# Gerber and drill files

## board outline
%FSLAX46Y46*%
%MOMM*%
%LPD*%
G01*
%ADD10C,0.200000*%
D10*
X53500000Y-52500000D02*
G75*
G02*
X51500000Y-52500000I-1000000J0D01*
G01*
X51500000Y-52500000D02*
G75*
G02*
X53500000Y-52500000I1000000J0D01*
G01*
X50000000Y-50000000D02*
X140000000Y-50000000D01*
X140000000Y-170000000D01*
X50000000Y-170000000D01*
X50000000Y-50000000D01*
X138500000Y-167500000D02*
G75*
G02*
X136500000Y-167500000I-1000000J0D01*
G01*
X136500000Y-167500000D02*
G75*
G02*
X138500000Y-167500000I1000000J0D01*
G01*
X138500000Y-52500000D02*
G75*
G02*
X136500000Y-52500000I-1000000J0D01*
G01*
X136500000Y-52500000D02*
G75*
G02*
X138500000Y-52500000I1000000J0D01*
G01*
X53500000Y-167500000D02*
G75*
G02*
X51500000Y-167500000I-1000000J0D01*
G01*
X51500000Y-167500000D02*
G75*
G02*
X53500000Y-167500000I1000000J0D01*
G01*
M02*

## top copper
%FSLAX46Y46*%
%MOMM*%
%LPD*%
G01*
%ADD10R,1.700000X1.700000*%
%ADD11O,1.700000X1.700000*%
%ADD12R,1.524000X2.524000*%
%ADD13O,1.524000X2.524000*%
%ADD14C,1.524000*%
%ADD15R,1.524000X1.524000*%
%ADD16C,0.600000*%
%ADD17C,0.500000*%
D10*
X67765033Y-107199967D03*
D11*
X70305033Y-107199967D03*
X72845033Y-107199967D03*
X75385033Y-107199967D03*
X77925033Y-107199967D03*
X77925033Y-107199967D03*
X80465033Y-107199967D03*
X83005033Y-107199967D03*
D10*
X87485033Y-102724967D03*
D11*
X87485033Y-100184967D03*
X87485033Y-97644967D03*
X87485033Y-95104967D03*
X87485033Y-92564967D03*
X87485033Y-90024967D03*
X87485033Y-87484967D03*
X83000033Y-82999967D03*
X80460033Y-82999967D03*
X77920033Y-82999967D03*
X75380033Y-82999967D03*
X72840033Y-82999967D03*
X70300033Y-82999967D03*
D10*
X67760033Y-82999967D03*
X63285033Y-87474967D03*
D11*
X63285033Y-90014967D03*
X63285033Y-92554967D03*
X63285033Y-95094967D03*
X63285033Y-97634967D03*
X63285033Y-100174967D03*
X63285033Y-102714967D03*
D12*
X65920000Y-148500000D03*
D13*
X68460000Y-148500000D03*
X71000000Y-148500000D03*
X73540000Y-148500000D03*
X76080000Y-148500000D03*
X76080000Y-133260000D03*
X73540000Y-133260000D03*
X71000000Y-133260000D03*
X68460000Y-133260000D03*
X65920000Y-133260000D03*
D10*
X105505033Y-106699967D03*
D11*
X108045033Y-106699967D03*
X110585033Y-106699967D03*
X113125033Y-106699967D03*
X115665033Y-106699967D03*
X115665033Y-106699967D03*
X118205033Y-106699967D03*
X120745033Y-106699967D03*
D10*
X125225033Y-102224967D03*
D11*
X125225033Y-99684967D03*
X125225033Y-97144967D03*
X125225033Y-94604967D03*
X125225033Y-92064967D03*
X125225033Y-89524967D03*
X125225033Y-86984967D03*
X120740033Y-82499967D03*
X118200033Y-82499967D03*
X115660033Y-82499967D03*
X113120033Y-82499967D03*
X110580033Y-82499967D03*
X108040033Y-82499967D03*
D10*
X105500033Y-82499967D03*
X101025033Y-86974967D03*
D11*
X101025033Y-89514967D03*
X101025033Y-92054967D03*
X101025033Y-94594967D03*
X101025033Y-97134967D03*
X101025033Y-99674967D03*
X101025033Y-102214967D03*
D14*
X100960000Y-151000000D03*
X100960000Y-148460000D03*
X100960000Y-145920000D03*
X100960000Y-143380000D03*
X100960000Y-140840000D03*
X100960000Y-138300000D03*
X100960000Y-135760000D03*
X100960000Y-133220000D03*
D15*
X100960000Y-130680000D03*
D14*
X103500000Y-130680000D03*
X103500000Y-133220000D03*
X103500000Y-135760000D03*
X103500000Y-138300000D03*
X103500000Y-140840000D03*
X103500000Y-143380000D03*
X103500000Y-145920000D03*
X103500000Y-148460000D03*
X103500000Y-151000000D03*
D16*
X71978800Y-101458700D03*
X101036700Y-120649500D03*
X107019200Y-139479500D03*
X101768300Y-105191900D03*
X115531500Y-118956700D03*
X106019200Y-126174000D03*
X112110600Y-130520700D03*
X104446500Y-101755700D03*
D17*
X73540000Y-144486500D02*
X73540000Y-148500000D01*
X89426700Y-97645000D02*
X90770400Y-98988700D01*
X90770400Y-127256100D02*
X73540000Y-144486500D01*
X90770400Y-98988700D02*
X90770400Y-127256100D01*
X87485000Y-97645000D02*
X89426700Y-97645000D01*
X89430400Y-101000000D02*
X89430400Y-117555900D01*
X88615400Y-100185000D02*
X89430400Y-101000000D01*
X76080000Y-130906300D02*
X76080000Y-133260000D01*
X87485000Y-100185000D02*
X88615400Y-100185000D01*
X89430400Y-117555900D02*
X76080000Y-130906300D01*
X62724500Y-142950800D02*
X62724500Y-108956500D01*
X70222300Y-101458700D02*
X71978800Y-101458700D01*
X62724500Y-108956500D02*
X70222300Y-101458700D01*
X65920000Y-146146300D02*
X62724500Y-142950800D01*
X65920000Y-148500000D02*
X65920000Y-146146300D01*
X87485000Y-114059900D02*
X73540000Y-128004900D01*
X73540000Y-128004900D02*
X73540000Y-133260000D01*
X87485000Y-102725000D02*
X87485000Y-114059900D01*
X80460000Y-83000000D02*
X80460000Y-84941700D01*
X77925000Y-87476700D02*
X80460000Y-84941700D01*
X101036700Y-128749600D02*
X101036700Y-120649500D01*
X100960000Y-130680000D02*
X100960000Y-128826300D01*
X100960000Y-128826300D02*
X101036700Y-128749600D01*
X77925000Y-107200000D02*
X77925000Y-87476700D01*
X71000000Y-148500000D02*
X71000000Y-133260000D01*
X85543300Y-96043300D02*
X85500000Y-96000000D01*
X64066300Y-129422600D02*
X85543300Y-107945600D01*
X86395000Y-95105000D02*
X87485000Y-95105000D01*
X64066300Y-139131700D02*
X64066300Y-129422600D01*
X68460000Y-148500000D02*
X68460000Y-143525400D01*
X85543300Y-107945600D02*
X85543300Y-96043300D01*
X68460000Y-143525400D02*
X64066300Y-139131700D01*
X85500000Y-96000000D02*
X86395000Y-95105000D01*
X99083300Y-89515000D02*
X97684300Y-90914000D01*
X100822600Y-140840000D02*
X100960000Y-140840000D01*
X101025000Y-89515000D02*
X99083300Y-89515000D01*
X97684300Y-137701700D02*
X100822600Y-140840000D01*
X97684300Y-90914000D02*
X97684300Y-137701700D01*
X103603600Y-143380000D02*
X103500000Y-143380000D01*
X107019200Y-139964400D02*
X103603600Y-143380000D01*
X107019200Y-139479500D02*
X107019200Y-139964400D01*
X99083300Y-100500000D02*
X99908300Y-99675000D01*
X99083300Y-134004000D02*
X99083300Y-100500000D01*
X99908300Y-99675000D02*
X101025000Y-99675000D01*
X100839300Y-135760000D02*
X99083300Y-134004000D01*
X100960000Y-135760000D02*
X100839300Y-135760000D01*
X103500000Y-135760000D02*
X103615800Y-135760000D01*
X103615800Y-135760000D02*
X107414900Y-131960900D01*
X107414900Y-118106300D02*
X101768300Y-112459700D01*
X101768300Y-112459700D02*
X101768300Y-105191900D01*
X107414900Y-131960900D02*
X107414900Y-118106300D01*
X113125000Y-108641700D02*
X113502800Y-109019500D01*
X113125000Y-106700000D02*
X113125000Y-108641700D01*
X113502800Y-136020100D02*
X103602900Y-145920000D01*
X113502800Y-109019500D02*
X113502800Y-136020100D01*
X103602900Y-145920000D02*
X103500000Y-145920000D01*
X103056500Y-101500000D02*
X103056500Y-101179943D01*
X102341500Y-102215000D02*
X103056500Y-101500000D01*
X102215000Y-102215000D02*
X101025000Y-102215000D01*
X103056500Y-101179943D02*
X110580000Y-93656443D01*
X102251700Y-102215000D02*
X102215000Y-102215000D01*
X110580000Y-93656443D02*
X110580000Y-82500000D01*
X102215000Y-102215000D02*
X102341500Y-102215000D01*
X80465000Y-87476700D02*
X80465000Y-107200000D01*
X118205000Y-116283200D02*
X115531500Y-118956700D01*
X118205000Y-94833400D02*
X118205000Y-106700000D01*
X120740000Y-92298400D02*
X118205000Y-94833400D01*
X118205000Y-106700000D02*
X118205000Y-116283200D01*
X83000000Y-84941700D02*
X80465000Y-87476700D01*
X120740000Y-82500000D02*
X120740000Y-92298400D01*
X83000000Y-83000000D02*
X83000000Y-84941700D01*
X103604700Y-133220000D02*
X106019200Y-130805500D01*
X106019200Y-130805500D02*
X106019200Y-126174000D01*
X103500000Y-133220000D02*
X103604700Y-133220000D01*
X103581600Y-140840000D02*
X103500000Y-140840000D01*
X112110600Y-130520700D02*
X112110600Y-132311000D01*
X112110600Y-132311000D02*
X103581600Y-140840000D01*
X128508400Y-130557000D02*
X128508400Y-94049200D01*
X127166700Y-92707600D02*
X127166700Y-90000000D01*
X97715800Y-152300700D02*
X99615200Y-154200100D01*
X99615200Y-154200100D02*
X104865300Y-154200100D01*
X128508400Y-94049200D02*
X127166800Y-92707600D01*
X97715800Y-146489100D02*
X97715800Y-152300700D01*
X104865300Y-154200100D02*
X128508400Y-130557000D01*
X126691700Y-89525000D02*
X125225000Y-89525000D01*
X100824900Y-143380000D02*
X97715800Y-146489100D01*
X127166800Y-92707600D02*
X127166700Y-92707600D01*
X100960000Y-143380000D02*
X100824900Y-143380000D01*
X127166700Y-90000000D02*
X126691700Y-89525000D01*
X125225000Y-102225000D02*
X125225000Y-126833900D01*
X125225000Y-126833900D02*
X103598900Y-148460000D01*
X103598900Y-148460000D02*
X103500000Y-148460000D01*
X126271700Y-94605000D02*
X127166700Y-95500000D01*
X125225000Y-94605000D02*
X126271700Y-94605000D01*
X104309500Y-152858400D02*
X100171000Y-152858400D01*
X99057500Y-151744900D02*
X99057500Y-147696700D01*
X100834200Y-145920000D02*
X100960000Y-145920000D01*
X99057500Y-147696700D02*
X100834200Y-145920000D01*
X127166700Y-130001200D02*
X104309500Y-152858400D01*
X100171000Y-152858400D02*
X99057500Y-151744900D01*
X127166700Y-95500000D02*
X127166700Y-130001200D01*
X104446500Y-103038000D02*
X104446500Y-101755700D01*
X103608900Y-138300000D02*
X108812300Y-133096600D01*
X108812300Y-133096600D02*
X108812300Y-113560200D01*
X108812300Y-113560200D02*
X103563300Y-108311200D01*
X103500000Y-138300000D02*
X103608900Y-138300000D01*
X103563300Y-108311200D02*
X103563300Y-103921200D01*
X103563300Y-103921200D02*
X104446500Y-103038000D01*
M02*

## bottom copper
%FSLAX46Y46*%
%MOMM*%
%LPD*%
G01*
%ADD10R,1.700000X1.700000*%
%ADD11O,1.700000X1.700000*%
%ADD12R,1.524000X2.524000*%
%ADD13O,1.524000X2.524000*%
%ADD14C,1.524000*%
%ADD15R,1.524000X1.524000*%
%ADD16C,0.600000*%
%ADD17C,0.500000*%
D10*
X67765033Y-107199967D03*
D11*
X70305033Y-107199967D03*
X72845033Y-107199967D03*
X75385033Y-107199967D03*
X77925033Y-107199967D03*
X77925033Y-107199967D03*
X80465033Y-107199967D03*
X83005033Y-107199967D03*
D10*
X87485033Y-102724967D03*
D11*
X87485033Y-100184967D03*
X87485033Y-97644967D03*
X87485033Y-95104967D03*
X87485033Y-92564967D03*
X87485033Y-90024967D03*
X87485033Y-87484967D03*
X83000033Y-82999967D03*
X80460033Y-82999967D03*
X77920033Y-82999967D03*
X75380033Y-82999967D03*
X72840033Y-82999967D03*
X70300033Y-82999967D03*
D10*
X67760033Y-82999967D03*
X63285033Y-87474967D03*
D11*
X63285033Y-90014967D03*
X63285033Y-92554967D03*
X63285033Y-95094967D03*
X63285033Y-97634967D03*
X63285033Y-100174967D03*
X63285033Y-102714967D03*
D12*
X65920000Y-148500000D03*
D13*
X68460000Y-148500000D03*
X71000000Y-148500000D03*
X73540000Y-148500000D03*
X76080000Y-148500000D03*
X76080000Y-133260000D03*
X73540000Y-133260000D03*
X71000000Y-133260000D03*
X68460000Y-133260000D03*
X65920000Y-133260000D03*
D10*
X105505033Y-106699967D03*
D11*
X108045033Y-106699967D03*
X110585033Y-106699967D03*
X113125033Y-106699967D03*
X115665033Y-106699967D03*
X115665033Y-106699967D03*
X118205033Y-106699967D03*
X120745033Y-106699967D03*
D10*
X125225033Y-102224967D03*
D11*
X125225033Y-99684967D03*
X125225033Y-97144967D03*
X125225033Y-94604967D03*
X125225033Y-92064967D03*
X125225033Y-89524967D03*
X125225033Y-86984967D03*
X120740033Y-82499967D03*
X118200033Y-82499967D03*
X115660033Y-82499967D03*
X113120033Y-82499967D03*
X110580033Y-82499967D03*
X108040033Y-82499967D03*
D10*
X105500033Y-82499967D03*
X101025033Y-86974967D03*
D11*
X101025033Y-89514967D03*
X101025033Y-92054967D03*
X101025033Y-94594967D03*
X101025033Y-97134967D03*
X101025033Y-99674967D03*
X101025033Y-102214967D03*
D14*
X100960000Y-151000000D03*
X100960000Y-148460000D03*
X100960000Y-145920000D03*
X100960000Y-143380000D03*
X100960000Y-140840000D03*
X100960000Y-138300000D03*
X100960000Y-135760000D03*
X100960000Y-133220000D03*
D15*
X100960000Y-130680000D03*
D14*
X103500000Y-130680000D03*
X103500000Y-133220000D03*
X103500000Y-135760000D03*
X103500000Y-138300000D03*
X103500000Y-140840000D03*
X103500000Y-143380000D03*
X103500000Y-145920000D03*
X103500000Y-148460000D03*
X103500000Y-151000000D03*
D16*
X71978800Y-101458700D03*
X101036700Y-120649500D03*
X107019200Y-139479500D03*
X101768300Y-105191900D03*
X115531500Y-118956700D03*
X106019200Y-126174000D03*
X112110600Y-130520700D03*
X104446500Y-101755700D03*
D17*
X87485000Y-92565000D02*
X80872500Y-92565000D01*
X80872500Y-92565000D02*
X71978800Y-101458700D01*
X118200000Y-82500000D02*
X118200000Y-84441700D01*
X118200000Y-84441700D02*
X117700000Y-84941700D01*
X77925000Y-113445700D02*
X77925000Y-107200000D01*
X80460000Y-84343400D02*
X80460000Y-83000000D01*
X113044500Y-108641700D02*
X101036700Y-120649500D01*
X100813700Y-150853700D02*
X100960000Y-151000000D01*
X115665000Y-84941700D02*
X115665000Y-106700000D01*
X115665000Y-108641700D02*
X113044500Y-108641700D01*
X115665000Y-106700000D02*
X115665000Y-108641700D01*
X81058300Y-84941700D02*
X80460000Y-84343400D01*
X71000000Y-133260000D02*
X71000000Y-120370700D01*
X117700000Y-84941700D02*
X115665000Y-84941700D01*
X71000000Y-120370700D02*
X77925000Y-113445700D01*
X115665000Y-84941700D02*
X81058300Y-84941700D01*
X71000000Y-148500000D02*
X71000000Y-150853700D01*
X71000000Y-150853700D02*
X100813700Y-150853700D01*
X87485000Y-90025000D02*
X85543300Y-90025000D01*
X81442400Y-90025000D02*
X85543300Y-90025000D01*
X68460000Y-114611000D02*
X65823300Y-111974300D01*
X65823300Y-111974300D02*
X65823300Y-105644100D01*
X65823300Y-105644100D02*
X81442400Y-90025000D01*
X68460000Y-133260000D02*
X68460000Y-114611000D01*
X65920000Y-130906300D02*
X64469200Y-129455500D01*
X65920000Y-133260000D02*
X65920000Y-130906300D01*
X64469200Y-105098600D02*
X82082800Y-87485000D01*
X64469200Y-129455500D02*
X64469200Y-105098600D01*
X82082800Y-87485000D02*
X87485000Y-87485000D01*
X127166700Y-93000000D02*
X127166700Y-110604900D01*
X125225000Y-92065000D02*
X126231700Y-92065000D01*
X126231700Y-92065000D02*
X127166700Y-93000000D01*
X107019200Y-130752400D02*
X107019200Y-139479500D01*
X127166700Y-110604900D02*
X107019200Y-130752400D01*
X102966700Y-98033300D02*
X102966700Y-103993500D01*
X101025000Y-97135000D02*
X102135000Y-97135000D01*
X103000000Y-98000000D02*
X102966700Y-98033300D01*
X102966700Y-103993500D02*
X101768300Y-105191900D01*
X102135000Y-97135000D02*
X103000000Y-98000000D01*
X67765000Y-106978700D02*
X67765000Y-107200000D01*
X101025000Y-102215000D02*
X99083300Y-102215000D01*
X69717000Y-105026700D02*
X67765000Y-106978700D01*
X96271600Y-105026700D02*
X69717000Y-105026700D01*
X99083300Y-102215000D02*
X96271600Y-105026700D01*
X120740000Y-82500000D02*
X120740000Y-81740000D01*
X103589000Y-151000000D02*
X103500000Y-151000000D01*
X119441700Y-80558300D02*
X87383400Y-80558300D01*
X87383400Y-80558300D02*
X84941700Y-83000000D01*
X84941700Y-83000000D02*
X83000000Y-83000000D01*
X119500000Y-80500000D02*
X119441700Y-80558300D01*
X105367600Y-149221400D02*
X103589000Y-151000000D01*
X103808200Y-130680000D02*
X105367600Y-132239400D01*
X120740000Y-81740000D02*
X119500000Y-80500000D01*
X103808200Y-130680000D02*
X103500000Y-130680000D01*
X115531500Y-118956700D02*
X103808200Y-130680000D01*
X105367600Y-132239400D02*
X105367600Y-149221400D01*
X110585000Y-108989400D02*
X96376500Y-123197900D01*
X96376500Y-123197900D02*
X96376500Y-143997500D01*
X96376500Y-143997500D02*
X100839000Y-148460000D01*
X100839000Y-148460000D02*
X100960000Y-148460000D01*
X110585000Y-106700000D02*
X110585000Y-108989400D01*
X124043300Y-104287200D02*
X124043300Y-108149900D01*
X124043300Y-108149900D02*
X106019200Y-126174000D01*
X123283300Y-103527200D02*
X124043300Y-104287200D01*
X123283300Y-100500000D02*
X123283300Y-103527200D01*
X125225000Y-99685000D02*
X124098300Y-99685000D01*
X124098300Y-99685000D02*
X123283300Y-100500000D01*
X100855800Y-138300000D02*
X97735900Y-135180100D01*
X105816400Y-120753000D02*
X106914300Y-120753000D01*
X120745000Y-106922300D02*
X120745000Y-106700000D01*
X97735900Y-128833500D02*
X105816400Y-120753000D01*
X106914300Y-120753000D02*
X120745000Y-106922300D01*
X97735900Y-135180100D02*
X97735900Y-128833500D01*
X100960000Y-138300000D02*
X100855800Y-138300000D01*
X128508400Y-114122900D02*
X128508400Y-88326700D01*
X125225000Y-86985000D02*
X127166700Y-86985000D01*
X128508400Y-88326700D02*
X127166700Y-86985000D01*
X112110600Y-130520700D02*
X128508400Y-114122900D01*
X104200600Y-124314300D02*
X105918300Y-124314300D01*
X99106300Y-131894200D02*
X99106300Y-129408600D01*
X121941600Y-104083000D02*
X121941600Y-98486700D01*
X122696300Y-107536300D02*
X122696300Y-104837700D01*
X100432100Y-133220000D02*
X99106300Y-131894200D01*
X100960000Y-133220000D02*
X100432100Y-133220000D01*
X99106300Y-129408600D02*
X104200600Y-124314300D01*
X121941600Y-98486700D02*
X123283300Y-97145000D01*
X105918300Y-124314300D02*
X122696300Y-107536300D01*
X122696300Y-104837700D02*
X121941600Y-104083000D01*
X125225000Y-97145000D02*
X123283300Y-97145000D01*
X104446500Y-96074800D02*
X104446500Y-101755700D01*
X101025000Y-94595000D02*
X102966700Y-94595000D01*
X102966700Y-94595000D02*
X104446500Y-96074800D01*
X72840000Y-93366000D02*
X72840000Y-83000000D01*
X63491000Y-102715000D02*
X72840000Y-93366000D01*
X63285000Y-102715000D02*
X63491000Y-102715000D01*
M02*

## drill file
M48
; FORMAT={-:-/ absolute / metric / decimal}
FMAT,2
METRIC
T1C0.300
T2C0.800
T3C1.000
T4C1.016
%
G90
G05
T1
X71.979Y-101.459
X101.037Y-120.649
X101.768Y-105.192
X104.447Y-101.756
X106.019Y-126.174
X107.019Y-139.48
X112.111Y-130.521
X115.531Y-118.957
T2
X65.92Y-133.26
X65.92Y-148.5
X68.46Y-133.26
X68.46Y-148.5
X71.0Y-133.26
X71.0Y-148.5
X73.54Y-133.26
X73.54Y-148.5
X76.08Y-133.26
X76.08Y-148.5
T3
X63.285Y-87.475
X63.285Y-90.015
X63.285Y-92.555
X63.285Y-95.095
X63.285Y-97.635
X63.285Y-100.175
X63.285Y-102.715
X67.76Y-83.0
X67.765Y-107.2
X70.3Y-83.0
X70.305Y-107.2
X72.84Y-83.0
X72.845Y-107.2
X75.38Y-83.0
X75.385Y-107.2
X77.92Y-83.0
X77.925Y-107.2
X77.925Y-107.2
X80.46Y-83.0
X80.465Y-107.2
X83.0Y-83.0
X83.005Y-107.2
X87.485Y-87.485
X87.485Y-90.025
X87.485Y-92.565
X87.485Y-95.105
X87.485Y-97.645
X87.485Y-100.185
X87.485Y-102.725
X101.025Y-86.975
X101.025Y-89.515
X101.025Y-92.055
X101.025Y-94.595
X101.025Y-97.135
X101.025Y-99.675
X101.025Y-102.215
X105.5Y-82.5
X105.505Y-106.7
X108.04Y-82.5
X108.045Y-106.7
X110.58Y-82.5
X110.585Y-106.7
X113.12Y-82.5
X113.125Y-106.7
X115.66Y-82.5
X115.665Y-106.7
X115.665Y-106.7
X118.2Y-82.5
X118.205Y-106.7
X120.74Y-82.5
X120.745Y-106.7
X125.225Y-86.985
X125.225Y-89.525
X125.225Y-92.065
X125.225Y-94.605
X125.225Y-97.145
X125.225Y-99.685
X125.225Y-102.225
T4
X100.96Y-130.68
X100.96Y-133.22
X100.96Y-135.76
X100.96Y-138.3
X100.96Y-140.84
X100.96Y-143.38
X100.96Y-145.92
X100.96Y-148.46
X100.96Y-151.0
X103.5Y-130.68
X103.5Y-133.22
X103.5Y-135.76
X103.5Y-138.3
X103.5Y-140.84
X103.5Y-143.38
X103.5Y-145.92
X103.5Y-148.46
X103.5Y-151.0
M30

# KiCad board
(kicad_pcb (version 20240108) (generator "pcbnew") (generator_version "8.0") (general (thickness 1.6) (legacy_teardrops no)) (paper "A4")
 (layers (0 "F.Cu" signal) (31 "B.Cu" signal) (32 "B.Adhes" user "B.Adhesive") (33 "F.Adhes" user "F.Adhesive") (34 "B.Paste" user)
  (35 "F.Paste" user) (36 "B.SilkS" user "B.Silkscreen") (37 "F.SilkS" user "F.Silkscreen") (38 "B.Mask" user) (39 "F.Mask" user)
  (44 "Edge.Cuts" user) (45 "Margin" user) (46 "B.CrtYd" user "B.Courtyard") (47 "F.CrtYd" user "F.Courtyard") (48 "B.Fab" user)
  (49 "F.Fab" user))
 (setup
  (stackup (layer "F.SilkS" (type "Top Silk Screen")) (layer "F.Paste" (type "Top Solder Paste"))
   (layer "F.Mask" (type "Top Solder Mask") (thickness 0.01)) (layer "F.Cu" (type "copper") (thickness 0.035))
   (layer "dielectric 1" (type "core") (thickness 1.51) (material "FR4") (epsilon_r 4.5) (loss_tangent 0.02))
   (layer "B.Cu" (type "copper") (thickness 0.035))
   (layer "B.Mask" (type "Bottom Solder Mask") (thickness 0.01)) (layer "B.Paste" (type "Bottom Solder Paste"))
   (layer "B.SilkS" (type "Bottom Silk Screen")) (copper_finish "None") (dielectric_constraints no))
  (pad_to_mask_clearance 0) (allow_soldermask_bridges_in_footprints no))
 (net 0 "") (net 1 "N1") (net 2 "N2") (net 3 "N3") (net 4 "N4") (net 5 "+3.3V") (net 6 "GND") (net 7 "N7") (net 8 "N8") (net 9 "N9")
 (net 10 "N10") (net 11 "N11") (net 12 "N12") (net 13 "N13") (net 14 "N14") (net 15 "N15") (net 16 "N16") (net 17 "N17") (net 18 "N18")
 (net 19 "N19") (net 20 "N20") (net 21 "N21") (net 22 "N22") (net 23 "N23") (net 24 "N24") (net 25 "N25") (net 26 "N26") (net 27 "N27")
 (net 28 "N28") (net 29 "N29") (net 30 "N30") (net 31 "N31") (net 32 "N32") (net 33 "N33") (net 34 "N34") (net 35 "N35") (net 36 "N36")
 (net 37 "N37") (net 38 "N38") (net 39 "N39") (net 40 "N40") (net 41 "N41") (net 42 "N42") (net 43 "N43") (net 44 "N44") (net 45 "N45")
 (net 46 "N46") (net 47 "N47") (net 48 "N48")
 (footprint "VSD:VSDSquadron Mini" (layer "F.Cu") (at 73.5486 95.2564 90)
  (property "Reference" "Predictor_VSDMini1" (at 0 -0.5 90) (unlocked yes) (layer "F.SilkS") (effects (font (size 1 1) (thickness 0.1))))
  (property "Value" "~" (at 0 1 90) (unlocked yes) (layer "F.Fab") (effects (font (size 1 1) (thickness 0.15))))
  (pad "1" thru_hole rect (at -11.943567 -5.783567 90) (size 1.7 1.7) (drill 1) (layers "*.Cu" "*.Mask") (remove_unused_layers no)
   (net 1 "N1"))
  (pad "2" thru_hole oval (at -11.943567 -3.243567 90) (size 1.7 1.7) (drill 1) (layers "*.Cu" "*.Mask") (remove_unused_layers no)
   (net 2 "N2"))
  (pad "3" thru_hole oval (at -11.943567 -0.703567 90) (size 1.7 1.7) (drill 1) (layers "*.Cu" "*.Mask") (remove_unused_layers no)
   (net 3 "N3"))
  (pad "4" thru_hole oval (at -11.943567 1.836433 90) (size 1.7 1.7) (drill 1) (layers "*.Cu" "*.Mask") (remove_unused_layers no)
   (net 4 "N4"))
  (pad "5" thru_hole oval (at -11.943567 4.376433 90) (size 1.7 1.7) (drill 1) (layers "*.Cu" "*.Mask") (remove_unused_layers no)
   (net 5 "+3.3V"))
  (pad "5" thru_hole oval (at -11.943567 4.376433 90) (size 1.7 1.7) (drill 1) (layers "*.Cu" "*.Mask") (remove_unused_layers no)
   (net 5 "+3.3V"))
  (pad "6" thru_hole oval (at -11.943567 6.916433 90) (size 1.7 1.7) (drill 1) (layers "*.Cu" "*.Mask") (remove_unused_layers no)
   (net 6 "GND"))
  (pad "7" thru_hole oval (at -11.943567 9.456433 90) (size 1.7 1.7) (drill 1) (layers "*.Cu" "*.Mask") (remove_unused_layers no)
   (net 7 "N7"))
  (pad "8" thru_hole rect (at -7.468567 13.936433 180) (size 1.7 1.7) (drill 1) (layers "*.Cu" "*.Mask") (remove_unused_layers no)
   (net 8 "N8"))
  (pad "9" thru_hole oval (at -4.928567 13.936433 180) (size 1.7 1.7) (drill 1) (layers "*.Cu" "*.Mask") (remove_unused_layers no)
   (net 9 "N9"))
  (pad "10" thru_hole oval (at -2.388567 13.936433 180) (size 1.7 1.7) (drill 1) (layers "*.Cu" "*.Mask") (remove_unused_layers no)
   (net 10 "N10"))
  (pad "11" thru_hole oval (at 0.151433 13.936433 180) (size 1.7 1.7) (drill 1) (layers "*.Cu" "*.Mask") (remove_unused_layers no)
   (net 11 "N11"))
  (pad "12" thru_hole oval (at 2.691433 13.936433 180) (size 1.7 1.7) (drill 1) (layers "*.Cu" "*.Mask") (remove_unused_layers no)
   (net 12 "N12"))
  (pad "13" thru_hole oval (at 5.231433 13.936433 180) (size 1.7 1.7) (drill 1) (layers "*.Cu" "*.Mask") (remove_unused_layers no)
   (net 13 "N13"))
  (pad "14" thru_hole oval (at 7.771433 13.936433 180) (size 1.7 1.7) (drill 1) (layers "*.Cu" "*.Mask") (remove_unused_layers no)
   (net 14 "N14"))
  (pad "15" thru_hole oval (at 12.256433 9.451433 90) (size 1.7 1.7) (drill 1) (layers "*.Cu" "*.Mask") (remove_unused_layers no)
   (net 6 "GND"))
  (pad "16" thru_hole oval (at 12.256433 6.911433 90) (size 1.7 1.7) (drill 1) (layers "*.Cu" "*.Mask") (remove_unused_layers no)
   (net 5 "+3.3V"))
  (pad "17" thru_hole oval (at 12.256433 4.371433 90) (size 1.7 1.7) (drill 1) (layers "*.Cu" "*.Mask") (remove_unused_layers no)
   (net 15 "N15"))
  (pad "18" thru_hole oval (at 12.256433 1.831433 90) (size 1.7 1.7) (drill 1) (layers "*.Cu" "*.Mask") (remove_unused_layers no)
   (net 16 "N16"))
  (pad "19" thru_hole oval (at 12.256433 -0.708567 90) (size 1.7 1.7) (drill 1) (layers "*.Cu" "*.Mask") (remove_unused_layers no)
   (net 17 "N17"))
  (pad "20" thru_hole oval (at 12.256433 -3.248567 90) (size 1.7 1.7) (drill 1) (layers "*.Cu" "*.Mask") (remove_unused_layers no)
   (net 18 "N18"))
  (pad "21" thru_hole rect (at 12.256433 -5.788567 90) (size 1.7 1.7) (drill 1) (layers "*.Cu" "*.Mask") (remove_unused_layers no)
   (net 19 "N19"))
  (pad "22" thru_hole rect (at 7.781433 -10.263567) (size 1.7 1.7) (drill 1) (layers "*.Cu" "*.Mask") (remove_unused_layers no)
   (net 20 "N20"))
  (pad "23" thru_hole oval (at 5.241433 -10.263567) (size 1.7 1.7) (drill 1) (layers "*.Cu" "*.Mask") (remove_unused_layers no)
   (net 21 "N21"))
  (pad "24" thru_hole oval (at 2.701433 -10.263567) (size 1.7 1.7) (drill 1) (layers "*.Cu" "*.Mask") (remove_unused_layers no)
   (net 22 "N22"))
  (pad "25" thru_hole oval (at 0.161433 -10.263567) (size 1.7 1.7) (drill 1) (layers "*.Cu" "*.Mask") (remove_unused_layers no)
   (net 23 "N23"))
  (pad "26" thru_hole oval (at -2.378567 -10.263567) (size 1.7 1.7) (drill 1) (layers "*.Cu" "*.Mask") (remove_unused_layers no)
   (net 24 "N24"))
  (pad "27" thru_hole oval (at -4.918567 -10.263567) (size 1.7 1.7) (drill 1) (layers "*.Cu" "*.Mask") (remove_unused_layers no)
   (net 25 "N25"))
  (pad "28" thru_hole oval (at -7.458567 -10.263567) (size 1.7 1.7) (drill 1) (layers "*.Cu" "*.Mask") (remove_unused_layers no)
   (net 17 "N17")))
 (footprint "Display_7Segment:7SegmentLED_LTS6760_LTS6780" (layer "F.Cu") (at 65.92 148.5 90)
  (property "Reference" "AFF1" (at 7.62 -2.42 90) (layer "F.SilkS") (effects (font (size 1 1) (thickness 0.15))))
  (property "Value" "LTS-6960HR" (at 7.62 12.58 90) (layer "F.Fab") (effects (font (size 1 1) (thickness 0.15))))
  (pad "1" thru_hole rect (at 0 0) (size 1.524 2.524) (drill 0.8) (layers "*.Cu" "*.Mask") (remove_unused_layers no) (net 12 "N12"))
  (pad "2" thru_hole oval (at 0 2.54) (size 1.524 2.524) (drill 0.8) (layers "*.Cu" "*.Mask") (remove_unused_layers no) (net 11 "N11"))
  (pad "3" thru_hole oval (at 0 5.08) (size 1.524 2.524) (drill 0.8) (layers "*.Cu" "*.Mask") (remove_unused_layers no) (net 5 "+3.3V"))
  (pad "4" thru_hole oval (at 0 7.62) (size 1.524 2.524) (drill 0.8) (layers "*.Cu" "*.Mask") (remove_unused_layers no) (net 10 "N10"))
  (pad "5" thru_hole oval (at 0 10.16) (size 1.524 2.524) (drill 0.8) (layers "*.Cu" "*.Mask") (remove_unused_layers no) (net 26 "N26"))
  (pad "6" thru_hole oval (at 15.24 10.16) (size 1.524 2.524) (drill 0.8) (layers "*.Cu" "*.Mask") (remove_unused_layers no) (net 9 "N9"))
  (pad "7" thru_hole oval (at 15.24 7.62) (size 1.524 2.524) (drill 0.8) (layers "*.Cu" "*.Mask") (remove_unused_layers no) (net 8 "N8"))
  (pad "8" thru_hole oval (at 15.24 5.08) (size 1.524 2.524) (drill 0.8) (layers "*.Cu" "*.Mask") (remove_unused_layers no) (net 5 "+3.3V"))
  (pad "9" thru_hole oval (at 15.24 2.54) (size 1.524 2.524) (drill 0.8) (layers "*.Cu" "*.Mask") (remove_unused_layers no) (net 13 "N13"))
  (pad "10" thru_hole oval (at 15.24 0) (size 1.524 2.524) (drill 0.8) (layers "*.Cu" "*.Mask") (remove_unused_layers no) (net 14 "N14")))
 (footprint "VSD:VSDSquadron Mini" (layer "F.Cu") (at 111.2886 94.7564 90)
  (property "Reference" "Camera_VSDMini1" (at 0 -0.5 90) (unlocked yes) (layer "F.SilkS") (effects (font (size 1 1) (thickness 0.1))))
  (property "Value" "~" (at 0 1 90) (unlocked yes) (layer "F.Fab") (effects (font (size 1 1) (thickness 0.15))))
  (pad "1" thru_hole rect (at -11.943567 -5.783567 90) (size 1.7 1.7) (drill 1) (layers "*.Cu" "*.Mask") (remove_unused_layers no)
   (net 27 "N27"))
  (pad "2" thru_hole oval (at -11.943567 -3.243567 90) (size 1.7 1.7) (drill 1) (layers "*.Cu" "*.Mask") (remove_unused_layers no)
   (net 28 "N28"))
  (pad "3" thru_hole oval (at -11.943567 -0.703567 90) (size 1.7 1.7) (drill 1) (layers "*.Cu" "*.Mask") (remove_unused_layers no)
   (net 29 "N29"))
  (pad "4" thru_hole oval (at -11.943567 1.836433 90) (size 1.7 1.7) (drill 1) (layers "*.Cu" "*.Mask") (remove_unused_layers no)
   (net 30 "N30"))
  (pad "5" thru_hole oval (at -11.943567 4.376433 90) (size 1.7 1.7) (drill 1) (layers "*.Cu" "*.Mask") (remove_unused_layers no)
   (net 5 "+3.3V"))
  (pad "5" thru_hole oval (at -11.943567 4.376433 90) (size 1.7 1.7) (drill 1) (layers "*.Cu" "*.Mask") (remove_unused_layers no)
   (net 5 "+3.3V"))
  (pad "6" thru_hole oval (at -11.943567 6.916433 90) (size 1.7 1.7) (drill 1) (layers "*.Cu" "*.Mask") (remove_unused_layers no)
   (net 6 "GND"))
  (pad "7" thru_hole oval (at -11.943567 9.456433 90) (size 1.7 1.7) (drill 1) (layers "*.Cu" "*.Mask") (remove_unused_layers no)
   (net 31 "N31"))
  (pad "8" thru_hole rect (at -7.468567 13.936433 180) (size 1.7 1.7) (drill 1) (layers "*.Cu" "*.Mask") (remove_unused_layers no)
   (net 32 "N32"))
  (pad "9" thru_hole oval (at -4.928567 13.936433 180) (size 1.7 1.7) (drill 1) (layers "*.Cu" "*.Mask") (remove_unused_layers no)
   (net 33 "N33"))
  (pad "10" thru_hole oval (at -2.388567 13.936433 180) (size 1.7 1.7) (drill 1) (layers "*.Cu" "*.Mask") (remove_unused_layers no)
   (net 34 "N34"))
  (pad "11" thru_hole oval (at 0.151433 13.936433 180) (size 1.7 1.7) (drill 1) (layers "*.Cu" "*.Mask") (remove_unused_layers no)
   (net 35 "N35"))
  (pad "12" thru_hole oval (at 2.691433 13.936433 180) (size 1.7 1.7) (drill 1) (layers "*.Cu" "*.Mask") (remove_unused_layers no)
   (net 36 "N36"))
  (pad "13" thru_hole oval (at 5.231433 13.936433 180) (size 1.7 1.7) (drill 1) (layers "*.Cu" "*.Mask") (remove_unused_layers no)
   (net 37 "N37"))
  (pad "14" thru_hole oval (at 7.771433 13.936433 180) (size 1.7 1.7) (drill 1) (layers "*.Cu" "*.Mask") (remove_unused_layers no)
   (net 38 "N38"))
  (pad "15" thru_hole oval (at 12.256433 9.451433 90) (size 1.7 1.7) (drill 1) (layers "*.Cu" "*.Mask") (remove_unused_layers no)
   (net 6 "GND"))
  (pad "16" thru_hole oval (at 12.256433 6.911433 90) (size 1.7 1.7) (drill 1) (layers "*.Cu" "*.Mask") (remove_unused_layers no)
   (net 5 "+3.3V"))
  (pad "17" thru_hole oval (at 12.256433 4.371433 90) (size 1.7 1.7) (drill 1) (layers "*.Cu" "*.Mask") (remove_unused_layers no)
   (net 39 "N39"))
  (pad "18" thru_hole oval (at 12.256433 1.831433 90) (size 1.7 1.7) (drill 1) (layers "*.Cu" "*.Mask") (remove_unused_layers no)
   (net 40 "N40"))
  (pad "19" thru_hole oval (at 12.256433 -0.708567 90) (size 1.7 1.7) (drill 1) (layers "*.Cu" "*.Mask") (remove_unused_layers no)
   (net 1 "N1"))
  (pad "20" thru_hole oval (at 12.256433 -3.248567 90) (size 1.7 1.7) (drill 1) (layers "*.Cu" "*.Mask") (remove_unused_layers no)
   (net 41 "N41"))
  (pad "21" thru_hole rect (at 12.256433 -5.788567 90) (size 1.7 1.7) (drill 1) (layers "*.Cu" "*.Mask") (remove_unused_layers no)
   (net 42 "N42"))
  (pad "22" thru_hole rect (at 7.781433 -10.263567) (size 1.7 1.7) (drill 1) (layers "*.Cu" "*.Mask") (remove_unused_layers no)
   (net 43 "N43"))
  (pad "23" thru_hole oval (at 5.241433 -10.263567) (size 1.7 1.7) (drill 1) (layers "*.Cu" "*.Mask") (remove_unused_layers no)
   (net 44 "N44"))
  (pad "24" thru_hole oval (at 2.701433 -10.263567) (size 1.7 1.7) (drill 1) (layers "*.Cu" "*.Mask") (remove_unused_layers no)
   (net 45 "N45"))
  (pad "25" thru_hole oval (at 0.161433 -10.263567) (size 1.7 1.7) (drill 1) (layers "*.Cu" "*.Mask") (remove_unused_layers no)
   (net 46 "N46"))
  (pad "26" thru_hole oval (at -2.378567 -10.263567) (size 1.7 1.7) (drill 1) (layers "*.Cu" "*.Mask") (remove_unused_layers no)
   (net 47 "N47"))
  (pad "27" thru_hole oval (at -4.918567 -10.263567) (size 1.7 1.7) (drill 1) (layers "*.Cu" "*.Mask") (remove_unused_layers no)
   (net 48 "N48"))
  (pad "28" thru_hole oval (at -7.458567 -10.263567) (size 1.7 1.7) (drill 1) (layers "*.Cu" "*.Mask") (remove_unused_layers no)
   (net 1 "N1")))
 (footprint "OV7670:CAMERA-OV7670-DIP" (layer "F.Cu") (at 114.46 141)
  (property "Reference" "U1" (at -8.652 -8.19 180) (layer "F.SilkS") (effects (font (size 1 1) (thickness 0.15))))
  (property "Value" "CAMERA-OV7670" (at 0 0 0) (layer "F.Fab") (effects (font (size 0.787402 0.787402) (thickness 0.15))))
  (pad "P$1" thru_hole circle (at -13.5 10) (size 1.524 1.524) (drill 1.016) (layers "*.Cu" "*.Mask") (remove_unused_layers no)
   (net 5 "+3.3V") (solder_mask_margin 0.102))
  (pad "P$2" thru_hole circle (at -13.5 7.46) (size 1.524 1.524) (drill 1.016) (layers "*.Cu" "*.Mask") (remove_unused_layers no)
   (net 29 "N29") (solder_mask_margin 0.102))
  (pad "P$3" thru_hole circle (at -13.5 4.92) (size 1.524 1.524) (drill 1.016) (layers "*.Cu" "*.Mask") (remove_unused_layers no)
   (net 35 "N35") (solder_mask_margin 0.102))
  (pad "P$4" thru_hole circle (at -13.5 2.38) (size 1.524 1.524) (drill 1.016) (layers "*.Cu" "*.Mask") (remove_unused_layers no)
   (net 37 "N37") (solder_mask_margin 0.102))
  (pad "P$5" thru_hole circle (at -13.5 -0.16) (size 1.524 1.524) (drill 1.016) (layers "*.Cu" "*.Mask") (remove_unused_layers no)
   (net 44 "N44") (solder_mask_margin 0.102))
  (pad "P$6" thru_hole circle (at -13.5 -2.7) (size 1.524 1.524) (drill 1.016) (layers "*.Cu" "*.Mask") (remove_unused_layers no)
   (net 31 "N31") (solder_mask_margin 0.102))
  (pad "P$7" thru_hole circle (at -13.5 -5.24) (size 1.524 1.524) (drill 1.016) (layers "*.Cu" "*.Mask") (remove_unused_layers no)
   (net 48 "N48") (solder_mask_margin 0.102))
  (pad "P$8" thru_hole circle (at -13.5 -7.78) (size 1.524 1.524) (drill 1.016) (layers "*.Cu" "*.Mask") (remove_unused_layers no)
   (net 34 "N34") (solder_mask_margin 0.102))
  (pad "P$9" thru_hole rect (at -13.5 -10.32) (size 1.524 1.524) (drill 1.016) (layers "*.Cu" "*.Mask") (remove_unused_layers no)
   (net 5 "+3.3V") (solder_mask_margin 0.102))
  (pad "P$10" thru_hole circle (at -10.96 -10.32) (size 1.524 1.524) (drill 1.016) (layers "*.Cu" "*.Mask") (remove_unused_layers no)
   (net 6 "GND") (solder_mask_margin 0.102))
  (pad "P$11" thru_hole circle (at -10.96 -7.78) (size 1.524 1.524) (drill 1.016) (layers "*.Cu" "*.Mask") (remove_unused_layers no)
   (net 33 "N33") (solder_mask_margin 0.102))
  (pad "P$12" thru_hole circle (at -10.96 -5.24) (size 1.524 1.524) (drill 1.016) (layers "*.Cu" "*.Mask") (remove_unused_layers no)
   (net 47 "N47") (solder_mask_margin 0.102))
  (pad "P$13" thru_hole circle (at -10.96 -2.7) (size 1.524 1.524) (drill 1.016) (layers "*.Cu" "*.Mask") (remove_unused_layers no)
   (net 46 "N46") (solder_mask_margin 0.102))
  (pad "P$14" thru_hole circle (at -10.96 -0.16) (size 1.524 1.524) (drill 1.016) (layers "*.Cu" "*.Mask") (remove_unused_layers no)
   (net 38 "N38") (solder_mask_margin 0.102))
  (pad "P$15" thru_hole circle (at -10.96 2.38) (size 1.524 1.524) (drill 1.016) (layers "*.Cu" "*.Mask") (remove_unused_layers no)
   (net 36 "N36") (solder_mask_margin 0.102))
  (pad "P$16" thru_hole circle (at -10.96 4.92) (size 1.524 1.524) (drill 1.016) (layers "*.Cu" "*.Mask") (remove_unused_layers no)
   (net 30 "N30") (solder_mask_margin 0.102))
  (pad "P$17" thru_hole circle (at -10.96 7.46) (size 1.524 1.524) (drill 1.016) (layers "*.Cu" "*.Mask") (remove_unused_layers no)
   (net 32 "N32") (solder_mask_margin 0.102))
  (pad "P$18" thru_hole circle (at -10.96 10) (size 1.524 1.524) (drill 1.016) (layers "*.Cu" "*.Mask") (remove_unused_layers no)
   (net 6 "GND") (solder_mask_margin 0.102)))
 (gr_circle (center 52.5 52.5) (end 52.5 53.5) (stroke (width 0.2) (type default)) (fill none) (layer "Edge.Cuts"))
 (gr_rect (start 50 50) (end 140 170) (stroke (width 0.2) (type default)) (fill none) (layer "Edge.Cuts"))
 (gr_circle (center 137.5 167.5) (end 137.5 168.5) (stroke (width 0.2) (type default)) (fill none) (layer "Edge.Cuts"))
 (gr_circle (center 137.5 52.5) (end 137.5 53.5) (stroke (width 0.2) (type default)) (fill none) (layer "Edge.Cuts"))
 (gr_circle (center 52.5 167.5) (end 52.5 168.5) (stroke (width 0.2) (type default)) (fill none) (layer "Edge.Cuts"))
 (segment (start 73.54 144.4865) (end 73.54 148.5) (width 0.5) (layer "F.Cu") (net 10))
 (segment (start 89.4267 97.645) (end 90.7704 98.9887) (width 0.5) (layer "F.Cu") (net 10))
 (segment (start 90.7704 127.2561) (end 73.54 144.4865) (width 0.5) (layer "F.Cu") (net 10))
 (segment (start 90.7704 98.9887) (end 90.7704 127.2561) (width 0.5) (layer "F.Cu") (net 10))
 (segment (start 87.485 97.645) (end 89.4267 97.645) (width 0.5) (layer "F.Cu") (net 10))
 (segment (start 89.4304 101) (end 89.4304 117.5559) (width 0.5) (layer "F.Cu") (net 9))
 (segment (start 88.6154 100.185) (end 89.4304 101) (width 0.5) (layer "F.Cu") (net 9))
 (segment (start 76.08 130.9063) (end 76.08 133.26) (width 0.5) (layer "F.Cu") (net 9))
 (segment (start 87.485 100.185) (end 88.6154 100.185) (width 0.5) (layer "F.Cu") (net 9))
 (segment (start 89.4304 117.5559) (end 76.08 130.9063) (width 0.5) (layer "F.Cu") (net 9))
 (segment (start 62.7245 142.9508) (end 62.7245 108.9565) (width 0.5) (layer "F.Cu") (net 12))
 (segment (start 70.2223 101.4587) (end 71.9788 101.4587) (width 0.5) (layer "F.Cu") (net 12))
 (segment (start 62.7245 108.9565) (end 70.2223 101.4587) (width 0.5) (layer "F.Cu") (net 12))
 (segment (start 65.92 146.1463) (end 62.7245 142.9508) (width 0.5) (layer "F.Cu") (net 12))
 (segment (start 65.92 148.5) (end 65.92 146.1463) (width 0.5) (layer "F.Cu") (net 12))
 (via (at 71.9788 101.4587) (size 0.6) (drill 0.3) (layers "F.Cu" "B.Cu") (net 12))
 (segment (start 87.485 92.565) (end 80.8725 92.565) (width 0.5) (layer "B.Cu") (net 12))
 (segment (start 80.8725 92.565) (end 71.9788 101.4587) (width 0.5) (layer "B.Cu") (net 12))
 (segment (start 87.485 114.0599) (end 73.54 128.0049) (width 0.5) (layer "F.Cu") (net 8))
 (segment (start 73.54 128.0049) (end 73.54 133.26) (width 0.5) (layer "F.Cu") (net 8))
 (segment (start 87.485 102.725) (end 87.485 114.0599) (width 0.5) (layer "F.Cu") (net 8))
 (segment (start 80.46 83) (end 80.46 84.9417) (width 0.5) (layer "F.Cu") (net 5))
 (segment (start 77.925 87.4767) (end 80.46 84.9417) (width 0.5) (layer "F.Cu") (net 5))
 (segment (start 101.0367 128.7496) (end 101.0367 120.6495) (width 0.5) (layer "F.Cu") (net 5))
 (segment (start 100.96 130.68) (end 100.96 128.8263) (width 0.5) (layer "F.Cu") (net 5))
 (segment (start 100.96 128.8263) (end 101.0367 128.7496) (width 0.5) (layer "F.Cu") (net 5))
 (segment (start 77.925 107.2) (end 77.925 87.4767) (width 0.5) (layer "F.Cu") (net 5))
 (segment (start 71 148.5) (end 71 133.26) (width 0.5) (layer "F.Cu") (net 5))
 (via (at 101.0367 120.6495) (size 0.6) (drill 0.3) (layers "F.Cu" "B.Cu") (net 5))
 (segment (start 118.2 82.5) (end 118.2 84.4417) (width 0.5) (layer "B.Cu") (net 5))
 (segment (start 118.2 84.4417) (end 117.7 84.9417) (width 0.5) (layer "B.Cu") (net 5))
 (segment (start 77.925 113.4457) (end 77.925 107.2) (width 0.5) (layer "B.Cu") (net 5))
 (segment (start 80.46 84.3434) (end 80.46 83) (width 0.5) (layer "B.Cu") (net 5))
 (segment (start 113.0445 108.6417) (end 101.0367 120.6495) (width 0.5) (layer "B.Cu") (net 5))
 (segment (start 100.8137 150.8537) (end 100.96 151) (width 0.5) (layer "B.Cu") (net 5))
 (segment (start 115.665 84.9417) (end 115.665 106.7) (width 0.5) (layer "B.Cu") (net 5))
 (segment (start 115.665 108.6417) (end 113.0445 108.6417) (width 0.5) (layer "B.Cu") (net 5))
 (segment (start 115.665 106.7) (end 115.665 108.6417) (width 0.5) (layer "B.Cu") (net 5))
 (segment (start 81.0583 84.9417) (end 80.46 84.3434) (width 0.5) (layer "B.Cu") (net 5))
 (segment (start 71 133.26) (end 71 120.3707) (width 0.5) (layer "B.Cu") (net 5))
 (segment (start 117.7 84.9417) (end 115.665 84.9417) (width 0.5) (layer "B.Cu") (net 5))
 (segment (start 71 120.3707) (end 77.925 113.4457) (width 0.5) (layer "B.Cu") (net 5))
 (segment (start 115.665 84.9417) (end 81.0583 84.9417) (width 0.5) (layer "B.Cu") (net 5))
 (segment (start 71 148.5) (end 71 150.8537) (width 0.5) (layer "B.Cu") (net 5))
 (segment (start 71 150.8537) (end 100.8137 150.8537) (width 0.5) (layer "B.Cu") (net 5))
 (segment (start 85.5433 96.0433) (end 85.5 96) (width 0.5) (layer "F.Cu") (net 11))
 (segment (start 64.0663 129.4226) (end 85.5433 107.9456) (width 0.5) (layer "F.Cu") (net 11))
 (segment (start 86.395 95.105) (end 87.485 95.105) (width 0.5) (layer "F.Cu") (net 11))
 (segment (start 64.0663 139.1317) (end 64.0663 129.4226) (width 0.5) (layer "F.Cu") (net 11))
 (segment (start 68.46 148.5) (end 68.46 143.5254) (width 0.5) (layer "F.Cu") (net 11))
 (segment (start 85.5433 107.9456) (end 85.5433 96.0433) (width 0.5) (layer "F.Cu") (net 11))
 (segment (start 68.46 143.5254) (end 64.0663 139.1317) (width 0.5) (layer "F.Cu") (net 11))
 (segment (start 85.5 96) (end 86.395 95.105) (width 0.5) (layer "F.Cu") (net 11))
 (segment (start 87.485 90.025) (end 85.5433 90.025) (width 0.5) (layer "B.Cu") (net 13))
 (segment (start 81.4424 90.025) (end 85.5433 90.025) (width 0.5) (layer "B.Cu") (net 13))
 (segment (start 68.46 114.611) (end 65.8233 111.9743) (width 0.5) (layer "B.Cu") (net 13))
 (segment (start 65.8233 111.9743) (end 65.8233 105.6441) (width 0.5) (layer "B.Cu") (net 13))
 (segment (start 65.8233 105.6441) (end 81.4424 90.025) (width 0.5) (layer "B.Cu") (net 13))
 (segment (start 68.46 133.26) (end 68.46 114.611) (width 0.5) (layer "B.Cu") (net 13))
 (segment (start 65.92 130.9063) (end 64.4692 129.4555) (width 0.5) (layer "B.Cu") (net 14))
 (segment (start 65.92 133.26) (end 65.92 130.9063) (width 0.5) (layer "B.Cu") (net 14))
 (segment (start 64.4692 105.0986) (end 82.0828 87.485) (width 0.5) (layer "B.Cu") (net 14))
 (segment (start 64.4692 129.4555) (end 64.4692 105.0986) (width 0.5) (layer "B.Cu") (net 14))
 (segment (start 82.0828 87.485) (end 87.485 87.485) (width 0.5) (layer "B.Cu") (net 14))
 (segment (start 99.0833 89.515) (end 97.6843 90.914) (width 0.5) (layer "F.Cu") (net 44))
 (segment (start 100.8226 140.84) (end 100.96 140.84) (width 0.5) (layer "F.Cu") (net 44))
 (segment (start 101.025 89.515) (end 99.0833 89.515) (width 0.5) (layer "F.Cu") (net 44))
 (segment (start 97.6843 137.7017) (end 100.8226 140.84) (width 0.5) (layer "F.Cu") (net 44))
 (segment (start 97.6843 90.914) (end 97.6843 137.7017) (width 0.5) (layer "F.Cu") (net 44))
 (segment (start 103.6036 143.38) (end 103.5 143.38) (width 0.5) (layer "F.Cu") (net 36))
 (segment (start 107.0192 139.9644) (end 103.6036 143.38) (width 0.5) (layer "F.Cu") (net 36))
 (segment (start 107.0192 139.4795) (end 107.0192 139.9644) (width 0.5) (layer "F.Cu") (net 36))
 (via (at 107.0192 139.4795) (size 0.6) (drill 0.3) (layers "F.Cu" "B.Cu") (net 36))
 (segment (start 127.1667 93) (end 127.1667 110.6049) (width 0.5) (layer "B.Cu") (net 36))
 (segment (start 125.225 92.065) (end 126.2317 92.065) (width 0.5) (layer "B.Cu") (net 36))
 (segment (start 126.2317 92.065) (end 127.1667 93) (width 0.5) (layer "B.Cu") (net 36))
 (segment (start 107.0192 130.7524) (end 107.0192 139.4795) (width 0.5) (layer "B.Cu") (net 36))
 (segment (start 127.1667 110.6049) (end 107.0192 130.7524) (width 0.5) (layer "B.Cu") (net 36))
 (segment (start 99.0833 100.5) (end 99.9083 99.675) (width 0.5) (layer "F.Cu") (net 48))
 (segment (start 99.0833 134.004) (end 99.0833 100.5) (width 0.5) (layer "F.Cu") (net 48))
 (segment (start 99.9083 99.675) (end 101.025 99.675) (width 0.5) (layer "F.Cu") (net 48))
 (segment (start 100.8393 135.76) (end 99.0833 134.004) (width 0.5) (layer "F.Cu") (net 48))
 (segment (start 100.96 135.76) (end 100.8393 135.76) (width 0.5) (layer "F.Cu") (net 48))
 (segment (start 103.5 135.76) (end 103.6158 135.76) (width 0.5) (layer "F.Cu") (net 47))
 (segment (start 103.6158 135.76) (end 107.4149 131.9609) (width 0.5) (layer "F.Cu") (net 47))
 (segment (start 107.4149 118.1063) (end 101.7683 112.4597) (width 0.5) (layer "F.Cu") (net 47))
 (segment (start 101.7683 112.4597) (end 101.7683 105.1919) (width 0.5) (layer "F.Cu") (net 47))
 (segment (start 107.4149 131.9609) (end 107.4149 118.1063) (width 0.5) (layer "F.Cu") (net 47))
 (via (at 101.7683 105.1919) (size 0.6) (drill 0.3) (layers "F.Cu" "B.Cu") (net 47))
 (segment (start 102.9667 98.0333) (end 102.9667 103.9935) (width 0.5) (layer "B.Cu") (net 47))
 (segment (start 101.025 97.135) (end 102.135 97.135) (width 0.5) (layer "B.Cu") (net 47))
 (segment (start 103 98) (end 102.9667 98.0333) (width 0.5) (layer "B.Cu") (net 47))
 (segment (start 102.9667 103.9935) (end 101.7683 105.1919) (width 0.5) (layer "B.Cu") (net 47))
 (segment (start 102.135 97.135) (end 103 98) (width 0.5) (layer "B.Cu") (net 47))
 (segment (start 113.125 108.6417) (end 113.5028 109.0195) (width 0.5) (layer "F.Cu") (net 30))
 (segment (start 113.125 106.7) (end 113.125 108.6417) (width 0.5) (layer "F.Cu") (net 30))
 (segment (start 113.5028 136.0201) (end 103.6029 145.92) (width 0.5) (layer "F.Cu") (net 30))
 (segment (start 113.5028 109.0195) (end 113.5028 136.0201) (width 0.5) (layer "F.Cu") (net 30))
 (segment (start 103.6029 145.92) (end 103.5 145.92) (width 0.5) (layer "F.Cu") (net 30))
 (segment (start 103.0565 101.5) (end 103.0565 101.179943) (width 0.5) (layer "F.Cu") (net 1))
 (segment (start 102.3415 102.215) (end 103.0565 101.5) (width 0.5) (layer "F.Cu") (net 1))
 (segment (start 102.215 102.215) (end 101.025 102.215) (width 0.5) (layer "F.Cu") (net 1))
 (segment (start 103.0565 101.179943) (end 110.58 93.656443) (width 0.5) (layer "F.Cu") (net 1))
 (segment (start 102.2517 102.215) (end 102.215 102.215) (width 0.5) (layer "F.Cu") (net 1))
 (segment (start 110.58 93.656443) (end 110.58 82.5) (width 0.5) (layer "F.Cu") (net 1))
 (segment (start 102.215 102.215) (end 102.3415 102.215) (width 0.5) (layer "F.Cu") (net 1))
 (segment (start 67.765 106.9787) (end 67.765 107.2) (width 0.5) (layer "B.Cu") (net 1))
 (segment (start 101.025 102.215) (end 99.0833 102.215) (width 0.5) (layer "B.Cu") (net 1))
 (segment (start 69.717 105.0267) (end 67.765 106.9787) (width 0.5) (layer "B.Cu") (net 1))
 (segment (start 96.2716 105.0267) (end 69.717 105.0267) (width 0.5) (layer "B.Cu") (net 1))
 (segment (start 99.0833 102.215) (end 96.2716 105.0267) (width 0.5) (layer "B.Cu") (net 1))
 (segment (start 80.465 87.4767) (end 80.465 107.2) (width 0.5) (layer "F.Cu") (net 6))
 (segment (start 118.205 116.2832) (end 115.5315 118.9567) (width 0.5) (layer "F.Cu") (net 6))
 (segment (start 118.205 94.8334) (end 118.205 106.7) (width 0.5) (layer "F.Cu") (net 6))
 (segment (start 120.74 92.2984) (end 118.205 94.8334) (width 0.5) (layer "F.Cu") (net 6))
 (segment (start 118.205 106.7) (end 118.205 116.2832) (width 0.5) (layer "F.Cu") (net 6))
 (segment (start 83 84.9417) (end 80.465 87.4767) (width 0.5) (layer "F.Cu") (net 6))
 (segment (start 120.74 82.5) (end 120.74 92.2984) (width 0.5) (layer "F.Cu") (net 6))
 (segment (start 83 83) (end 83 84.9417) (width 0.5) (layer "F.Cu") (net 6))
 (via (at 115.5315 118.9567) (size 0.6) (drill 0.3) (layers "F.Cu" "B.Cu") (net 6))
 (segment (start 120.74 82.5) (end 120.74 81.74) (width 0.5) (layer "B.Cu") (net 6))
 (segment (start 103.589 151) (end 103.5 151) (width 0.5) (layer "B.Cu") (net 6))
 (segment (start 119.4417 80.5583) (end 87.3834 80.5583) (width 0.5) (layer "B.Cu") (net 6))
 (segment (start 87.3834 80.5583) (end 84.9417 83) (width 0.5) (layer "B.Cu") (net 6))
 (segment (start 84.9417 83) (end 83 83) (width 0.5) (layer "B.Cu") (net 6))
 (segment (start 119.5 80.5) (end 119.4417 80.5583) (width 0.5) (layer "B.Cu") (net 6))
 (segment (start 105.3676 149.2214) (end 103.589 151) (width 0.5) (layer "B.Cu") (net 6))
 (segment (start 103.8082 130.68) (end 105.3676 132.2394) (width 0.5) (layer "B.Cu") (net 6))
 (segment (start 120.74 81.74) (end 119.5 80.5) (width 0.5) (layer "B.Cu") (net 6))
 (segment (start 103.8082 130.68) (end 103.5 130.68) (width 0.5) (layer "B.Cu") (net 6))
 (segment (start 115.5315 118.9567) (end 103.8082 130.68) (width 0.5) (layer "B.Cu") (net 6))
 (segment (start 105.3676 132.2394) (end 105.3676 149.2214) (width 0.5) (layer "B.Cu") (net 6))
 (segment (start 110.585 108.9894) (end 96.3765 123.1979) (width 0.5) (layer "B.Cu") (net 29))
 (segment (start 96.3765 123.1979) (end 96.3765 143.9975) (width 0.5) (layer "B.Cu") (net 29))
 (segment (start 96.3765 143.9975) (end 100.839 148.46) (width 0.5) (layer "B.Cu") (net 29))
 (segment (start 100.839 148.46) (end 100.96 148.46) (width 0.5) (layer "B.Cu") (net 29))
 (segment (start 110.585 106.7) (end 110.585 108.9894) (width 0.5) (layer "B.Cu") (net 29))
 (segment (start 103.6047 133.22) (end 106.0192 130.8055) (width 0.5) (layer "F.Cu") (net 33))
 (segment (start 106.0192 130.8055) (end 106.0192 126.174) (width 0.5) (layer "F.Cu") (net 33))
 (segment (start 103.5 133.22) (end 103.6047 133.22) (width 0.5) (layer "F.Cu") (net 33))
 (via (at 106.0192 126.174) (size 0.6) (drill 0.3) (layers "F.Cu" "B.Cu") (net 33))
 (segment (start 124.0433 104.2872) (end 124.0433 108.1499) (width 0.5) (layer "B.Cu") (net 33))
 (segment (start 124.0433 108.1499) (end 106.0192 126.174) (width 0.5) (layer "B.Cu") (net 33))
 (segment (start 123.2833 103.5272) (end 124.0433 104.2872) (width 0.5) (layer "B.Cu") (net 33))
 (segment (start 123.2833 100.5) (end 123.2833 103.5272) (width 0.5) (layer "B.Cu") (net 33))
 (segment (start 125.225 99.685) (end 124.0983 99.685) (width 0.5) (layer "B.Cu") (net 33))
 (segment (start 124.0983 99.685) (end 123.2833 100.5) (width 0.5) (layer "B.Cu") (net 33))
 (segment (start 100.8558 138.3) (end 97.7359 135.1801) (width 0.5) (layer "B.Cu") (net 31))
 (segment (start 105.8164 120.753) (end 106.9143 120.753) (width 0.5) (layer "B.Cu") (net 31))
 (segment (start 120.745 106.9223) (end 120.745 106.7) (width 0.5) (layer "B.Cu") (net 31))
 (segment (start 97.7359 128.8335) (end 105.8164 120.753) (width 0.5) (layer "B.Cu") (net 31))
 (segment (start 106.9143 120.753) (end 120.745 106.9223) (width 0.5) (layer "B.Cu") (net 31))
 (segment (start 97.7359 135.1801) (end 97.7359 128.8335) (width 0.5) (layer "B.Cu") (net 31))
 (segment (start 100.96 138.3) (end 100.8558 138.3) (width 0.5) (layer "B.Cu") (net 31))
 (segment (start 103.5816 140.84) (end 103.5 140.84) (width 0.5) (layer "F.Cu") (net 38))
 (segment (start 112.1106 130.5207) (end 112.1106 132.311) (width 0.5) (layer "F.Cu") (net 38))
 (segment (start 112.1106 132.311) (end 103.5816 140.84) (width 0.5) (layer "F.Cu") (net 38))
 (via (at 112.1106 130.5207) (size 0.6) (drill 0.3) (layers "F.Cu" "B.Cu") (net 38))
 (segment (start 128.5084 114.1229) (end 128.5084 88.3267) (width 0.5) (layer "B.Cu") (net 38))
 (segment (start 125.225 86.985) (end 127.1667 86.985) (width 0.5) (layer "B.Cu") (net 38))
 (segment (start 128.5084 88.3267) (end 127.1667 86.985) (width 0.5) (layer "B.Cu") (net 38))
 (segment (start 112.1106 130.5207) (end 128.5084 114.1229) (width 0.5) (layer "B.Cu") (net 38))
 (segment (start 104.2006 124.3143) (end 105.9183 124.3143) (width 0.5) (layer "B.Cu") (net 34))
 (segment (start 99.1063 131.8942) (end 99.1063 129.4086) (width 0.5) (layer "B.Cu") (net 34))
 (segment (start 121.9416 104.083) (end 121.9416 98.4867) (width 0.5) (layer "B.Cu") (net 34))
 (segment (start 122.6963 107.5363) (end 122.6963 104.8377) (width 0.5) (layer "B.Cu") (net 34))
 (segment (start 100.4321 133.22) (end 99.1063 131.8942) (width 0.5) (layer "B.Cu") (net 34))
 (segment (start 100.96 133.22) (end 100.4321 133.22) (width 0.5) (layer "B.Cu") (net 34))
 (segment (start 99.1063 129.4086) (end 104.2006 124.3143) (width 0.5) (layer "B.Cu") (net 34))
 (segment (start 121.9416 98.4867) (end 123.2833 97.145) (width 0.5) (layer "B.Cu") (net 34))
 (segment (start 105.9183 124.3143) (end 122.6963 107.5363) (width 0.5) (layer "B.Cu") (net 34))
 (segment (start 122.6963 104.8377) (end 121.9416 104.083) (width 0.5) (layer "B.Cu") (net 34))
 (segment (start 125.225 97.145) (end 123.2833 97.145) (width 0.5) (layer "B.Cu") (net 34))
 (segment (start 128.5084 130.557) (end 128.5084 94.0492) (width 0.5) (layer "F.Cu") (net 37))
 (segment (start 127.1667 92.7076) (end 127.1667 90) (width 0.5) (layer "F.Cu") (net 37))
 (segment (start 97.7158 152.3007) (end 99.6152 154.2001) (width 0.5) (layer "F.Cu") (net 37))
 (segment (start 99.6152 154.2001) (end 104.8653 154.2001) (width 0.5) (layer "F.Cu") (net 37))
 (segment (start 128.5084 94.0492) (end 127.1668 92.7076) (width 0.5) (layer "F.Cu") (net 37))
 (segment (start 97.7158 146.4891) (end 97.7158 152.3007) (width 0.5) (layer "F.Cu") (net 37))
 (segment (start 104.8653 154.2001) (end 128.5084 130.557) (width 0.5) (layer "F.Cu") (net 37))
 (segment (start 126.6917 89.525) (end 125.225 89.525) (width 0.5) (layer "F.Cu") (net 37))
 (segment (start 100.8249 143.38) (end 97.7158 146.4891) (width 0.5) (layer "F.Cu") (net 37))
 (segment (start 127.1668 92.7076) (end 127.1667 92.7076) (width 0.5) (layer "F.Cu") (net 37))
 (segment (start 100.96 143.38) (end 100.8249 143.38) (width 0.5) (layer "F.Cu") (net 37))
 (segment (start 127.1667 90) (end 126.6917 89.525) (width 0.5) (layer "F.Cu") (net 37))
 (segment (start 125.225 102.225) (end 125.225 126.8339) (width 0.5) (layer "F.Cu") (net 32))
 (segment (start 125.225 126.8339) (end 103.5989 148.46) (width 0.5) (layer "F.Cu") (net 32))
 (segment (start 103.5989 148.46) (end 103.5 148.46) (width 0.5) (layer "F.Cu") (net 32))
 (segment (start 126.2717 94.605) (end 127.1667 95.5) (width 0.5) (layer "F.Cu") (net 35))
 (segment (start 125.225 94.605) (end 126.2717 94.605) (width 0.5) (layer "F.Cu") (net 35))
 (segment (start 104.3095 152.8584) (end 100.171 152.8584) (width 0.5) (layer "F.Cu") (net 35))
 (segment (start 99.0575 151.7449) (end 99.0575 147.6967) (width 0.5) (layer "F.Cu") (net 35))
 (segment (start 100.8342 145.92) (end 100.96 145.92) (width 0.5) (layer "F.Cu") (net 35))
 (segment (start 99.0575 147.6967) (end 100.8342 145.92) (width 0.5) (layer "F.Cu") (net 35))
 (segment (start 127.1667 130.0012) (end 104.3095 152.8584) (width 0.5) (layer "F.Cu") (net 35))
 (segment (start 100.171 152.8584) (end 99.0575 151.7449) (width 0.5) (layer "F.Cu") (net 35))
 (segment (start 127.1667 95.5) (end 127.1667 130.0012) (width 0.5) (layer "F.Cu") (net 35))
 (segment (start 104.4465 103.038) (end 104.4465 101.7557) (width 0.5) (layer "F.Cu") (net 46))
 (segment (start 103.6089 138.3) (end 108.8123 133.0966) (width 0.5) (layer "F.Cu") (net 46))
 (segment (start 108.8123 133.0966) (end 108.8123 113.5602) (width 0.5) (layer "F.Cu") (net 46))
 (segment (start 108.8123 113.5602) (end 103.5633 108.3112) (width 0.5) (layer "F.Cu") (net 46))
 (segment (start 103.5 138.3) (end 103.6089 138.3) (width 0.5) (layer "F.Cu") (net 46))
 (segment (start 103.5633 108.3112) (end 103.5633 103.9212) (width 0.5) (layer "F.Cu") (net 46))
 (segment (start 103.5633 103.9212) (end 104.4465 103.038) (width 0.5) (layer "F.Cu") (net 46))
 (via (at 104.4465 101.7557) (size 0.6) (drill 0.3) (layers "F.Cu" "B.Cu") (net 46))
 (segment (start 104.4465 96.0748) (end 104.4465 101.7557) (width 0.5) (layer "B.Cu") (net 46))
 (segment (start 101.025 94.595) (end 102.9667 94.595) (width 0.5) (layer "B.Cu") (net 46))
 (segment (start 102.9667 94.595) (end 104.4465 96.0748) (width 0.5) (layer "B.Cu") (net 46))
 (segment (start 72.84 93.366) (end 72.84 83) (width 0.5) (layer "B.Cu") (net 17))
 (segment (start 63.491 102.715) (end 72.84 93.366) (width 0.5) (layer "B.Cu") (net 17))
 (segment (start 63.285 102.715) (end 63.491 102.715) (width 0.5) (layer "B.Cu") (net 17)))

